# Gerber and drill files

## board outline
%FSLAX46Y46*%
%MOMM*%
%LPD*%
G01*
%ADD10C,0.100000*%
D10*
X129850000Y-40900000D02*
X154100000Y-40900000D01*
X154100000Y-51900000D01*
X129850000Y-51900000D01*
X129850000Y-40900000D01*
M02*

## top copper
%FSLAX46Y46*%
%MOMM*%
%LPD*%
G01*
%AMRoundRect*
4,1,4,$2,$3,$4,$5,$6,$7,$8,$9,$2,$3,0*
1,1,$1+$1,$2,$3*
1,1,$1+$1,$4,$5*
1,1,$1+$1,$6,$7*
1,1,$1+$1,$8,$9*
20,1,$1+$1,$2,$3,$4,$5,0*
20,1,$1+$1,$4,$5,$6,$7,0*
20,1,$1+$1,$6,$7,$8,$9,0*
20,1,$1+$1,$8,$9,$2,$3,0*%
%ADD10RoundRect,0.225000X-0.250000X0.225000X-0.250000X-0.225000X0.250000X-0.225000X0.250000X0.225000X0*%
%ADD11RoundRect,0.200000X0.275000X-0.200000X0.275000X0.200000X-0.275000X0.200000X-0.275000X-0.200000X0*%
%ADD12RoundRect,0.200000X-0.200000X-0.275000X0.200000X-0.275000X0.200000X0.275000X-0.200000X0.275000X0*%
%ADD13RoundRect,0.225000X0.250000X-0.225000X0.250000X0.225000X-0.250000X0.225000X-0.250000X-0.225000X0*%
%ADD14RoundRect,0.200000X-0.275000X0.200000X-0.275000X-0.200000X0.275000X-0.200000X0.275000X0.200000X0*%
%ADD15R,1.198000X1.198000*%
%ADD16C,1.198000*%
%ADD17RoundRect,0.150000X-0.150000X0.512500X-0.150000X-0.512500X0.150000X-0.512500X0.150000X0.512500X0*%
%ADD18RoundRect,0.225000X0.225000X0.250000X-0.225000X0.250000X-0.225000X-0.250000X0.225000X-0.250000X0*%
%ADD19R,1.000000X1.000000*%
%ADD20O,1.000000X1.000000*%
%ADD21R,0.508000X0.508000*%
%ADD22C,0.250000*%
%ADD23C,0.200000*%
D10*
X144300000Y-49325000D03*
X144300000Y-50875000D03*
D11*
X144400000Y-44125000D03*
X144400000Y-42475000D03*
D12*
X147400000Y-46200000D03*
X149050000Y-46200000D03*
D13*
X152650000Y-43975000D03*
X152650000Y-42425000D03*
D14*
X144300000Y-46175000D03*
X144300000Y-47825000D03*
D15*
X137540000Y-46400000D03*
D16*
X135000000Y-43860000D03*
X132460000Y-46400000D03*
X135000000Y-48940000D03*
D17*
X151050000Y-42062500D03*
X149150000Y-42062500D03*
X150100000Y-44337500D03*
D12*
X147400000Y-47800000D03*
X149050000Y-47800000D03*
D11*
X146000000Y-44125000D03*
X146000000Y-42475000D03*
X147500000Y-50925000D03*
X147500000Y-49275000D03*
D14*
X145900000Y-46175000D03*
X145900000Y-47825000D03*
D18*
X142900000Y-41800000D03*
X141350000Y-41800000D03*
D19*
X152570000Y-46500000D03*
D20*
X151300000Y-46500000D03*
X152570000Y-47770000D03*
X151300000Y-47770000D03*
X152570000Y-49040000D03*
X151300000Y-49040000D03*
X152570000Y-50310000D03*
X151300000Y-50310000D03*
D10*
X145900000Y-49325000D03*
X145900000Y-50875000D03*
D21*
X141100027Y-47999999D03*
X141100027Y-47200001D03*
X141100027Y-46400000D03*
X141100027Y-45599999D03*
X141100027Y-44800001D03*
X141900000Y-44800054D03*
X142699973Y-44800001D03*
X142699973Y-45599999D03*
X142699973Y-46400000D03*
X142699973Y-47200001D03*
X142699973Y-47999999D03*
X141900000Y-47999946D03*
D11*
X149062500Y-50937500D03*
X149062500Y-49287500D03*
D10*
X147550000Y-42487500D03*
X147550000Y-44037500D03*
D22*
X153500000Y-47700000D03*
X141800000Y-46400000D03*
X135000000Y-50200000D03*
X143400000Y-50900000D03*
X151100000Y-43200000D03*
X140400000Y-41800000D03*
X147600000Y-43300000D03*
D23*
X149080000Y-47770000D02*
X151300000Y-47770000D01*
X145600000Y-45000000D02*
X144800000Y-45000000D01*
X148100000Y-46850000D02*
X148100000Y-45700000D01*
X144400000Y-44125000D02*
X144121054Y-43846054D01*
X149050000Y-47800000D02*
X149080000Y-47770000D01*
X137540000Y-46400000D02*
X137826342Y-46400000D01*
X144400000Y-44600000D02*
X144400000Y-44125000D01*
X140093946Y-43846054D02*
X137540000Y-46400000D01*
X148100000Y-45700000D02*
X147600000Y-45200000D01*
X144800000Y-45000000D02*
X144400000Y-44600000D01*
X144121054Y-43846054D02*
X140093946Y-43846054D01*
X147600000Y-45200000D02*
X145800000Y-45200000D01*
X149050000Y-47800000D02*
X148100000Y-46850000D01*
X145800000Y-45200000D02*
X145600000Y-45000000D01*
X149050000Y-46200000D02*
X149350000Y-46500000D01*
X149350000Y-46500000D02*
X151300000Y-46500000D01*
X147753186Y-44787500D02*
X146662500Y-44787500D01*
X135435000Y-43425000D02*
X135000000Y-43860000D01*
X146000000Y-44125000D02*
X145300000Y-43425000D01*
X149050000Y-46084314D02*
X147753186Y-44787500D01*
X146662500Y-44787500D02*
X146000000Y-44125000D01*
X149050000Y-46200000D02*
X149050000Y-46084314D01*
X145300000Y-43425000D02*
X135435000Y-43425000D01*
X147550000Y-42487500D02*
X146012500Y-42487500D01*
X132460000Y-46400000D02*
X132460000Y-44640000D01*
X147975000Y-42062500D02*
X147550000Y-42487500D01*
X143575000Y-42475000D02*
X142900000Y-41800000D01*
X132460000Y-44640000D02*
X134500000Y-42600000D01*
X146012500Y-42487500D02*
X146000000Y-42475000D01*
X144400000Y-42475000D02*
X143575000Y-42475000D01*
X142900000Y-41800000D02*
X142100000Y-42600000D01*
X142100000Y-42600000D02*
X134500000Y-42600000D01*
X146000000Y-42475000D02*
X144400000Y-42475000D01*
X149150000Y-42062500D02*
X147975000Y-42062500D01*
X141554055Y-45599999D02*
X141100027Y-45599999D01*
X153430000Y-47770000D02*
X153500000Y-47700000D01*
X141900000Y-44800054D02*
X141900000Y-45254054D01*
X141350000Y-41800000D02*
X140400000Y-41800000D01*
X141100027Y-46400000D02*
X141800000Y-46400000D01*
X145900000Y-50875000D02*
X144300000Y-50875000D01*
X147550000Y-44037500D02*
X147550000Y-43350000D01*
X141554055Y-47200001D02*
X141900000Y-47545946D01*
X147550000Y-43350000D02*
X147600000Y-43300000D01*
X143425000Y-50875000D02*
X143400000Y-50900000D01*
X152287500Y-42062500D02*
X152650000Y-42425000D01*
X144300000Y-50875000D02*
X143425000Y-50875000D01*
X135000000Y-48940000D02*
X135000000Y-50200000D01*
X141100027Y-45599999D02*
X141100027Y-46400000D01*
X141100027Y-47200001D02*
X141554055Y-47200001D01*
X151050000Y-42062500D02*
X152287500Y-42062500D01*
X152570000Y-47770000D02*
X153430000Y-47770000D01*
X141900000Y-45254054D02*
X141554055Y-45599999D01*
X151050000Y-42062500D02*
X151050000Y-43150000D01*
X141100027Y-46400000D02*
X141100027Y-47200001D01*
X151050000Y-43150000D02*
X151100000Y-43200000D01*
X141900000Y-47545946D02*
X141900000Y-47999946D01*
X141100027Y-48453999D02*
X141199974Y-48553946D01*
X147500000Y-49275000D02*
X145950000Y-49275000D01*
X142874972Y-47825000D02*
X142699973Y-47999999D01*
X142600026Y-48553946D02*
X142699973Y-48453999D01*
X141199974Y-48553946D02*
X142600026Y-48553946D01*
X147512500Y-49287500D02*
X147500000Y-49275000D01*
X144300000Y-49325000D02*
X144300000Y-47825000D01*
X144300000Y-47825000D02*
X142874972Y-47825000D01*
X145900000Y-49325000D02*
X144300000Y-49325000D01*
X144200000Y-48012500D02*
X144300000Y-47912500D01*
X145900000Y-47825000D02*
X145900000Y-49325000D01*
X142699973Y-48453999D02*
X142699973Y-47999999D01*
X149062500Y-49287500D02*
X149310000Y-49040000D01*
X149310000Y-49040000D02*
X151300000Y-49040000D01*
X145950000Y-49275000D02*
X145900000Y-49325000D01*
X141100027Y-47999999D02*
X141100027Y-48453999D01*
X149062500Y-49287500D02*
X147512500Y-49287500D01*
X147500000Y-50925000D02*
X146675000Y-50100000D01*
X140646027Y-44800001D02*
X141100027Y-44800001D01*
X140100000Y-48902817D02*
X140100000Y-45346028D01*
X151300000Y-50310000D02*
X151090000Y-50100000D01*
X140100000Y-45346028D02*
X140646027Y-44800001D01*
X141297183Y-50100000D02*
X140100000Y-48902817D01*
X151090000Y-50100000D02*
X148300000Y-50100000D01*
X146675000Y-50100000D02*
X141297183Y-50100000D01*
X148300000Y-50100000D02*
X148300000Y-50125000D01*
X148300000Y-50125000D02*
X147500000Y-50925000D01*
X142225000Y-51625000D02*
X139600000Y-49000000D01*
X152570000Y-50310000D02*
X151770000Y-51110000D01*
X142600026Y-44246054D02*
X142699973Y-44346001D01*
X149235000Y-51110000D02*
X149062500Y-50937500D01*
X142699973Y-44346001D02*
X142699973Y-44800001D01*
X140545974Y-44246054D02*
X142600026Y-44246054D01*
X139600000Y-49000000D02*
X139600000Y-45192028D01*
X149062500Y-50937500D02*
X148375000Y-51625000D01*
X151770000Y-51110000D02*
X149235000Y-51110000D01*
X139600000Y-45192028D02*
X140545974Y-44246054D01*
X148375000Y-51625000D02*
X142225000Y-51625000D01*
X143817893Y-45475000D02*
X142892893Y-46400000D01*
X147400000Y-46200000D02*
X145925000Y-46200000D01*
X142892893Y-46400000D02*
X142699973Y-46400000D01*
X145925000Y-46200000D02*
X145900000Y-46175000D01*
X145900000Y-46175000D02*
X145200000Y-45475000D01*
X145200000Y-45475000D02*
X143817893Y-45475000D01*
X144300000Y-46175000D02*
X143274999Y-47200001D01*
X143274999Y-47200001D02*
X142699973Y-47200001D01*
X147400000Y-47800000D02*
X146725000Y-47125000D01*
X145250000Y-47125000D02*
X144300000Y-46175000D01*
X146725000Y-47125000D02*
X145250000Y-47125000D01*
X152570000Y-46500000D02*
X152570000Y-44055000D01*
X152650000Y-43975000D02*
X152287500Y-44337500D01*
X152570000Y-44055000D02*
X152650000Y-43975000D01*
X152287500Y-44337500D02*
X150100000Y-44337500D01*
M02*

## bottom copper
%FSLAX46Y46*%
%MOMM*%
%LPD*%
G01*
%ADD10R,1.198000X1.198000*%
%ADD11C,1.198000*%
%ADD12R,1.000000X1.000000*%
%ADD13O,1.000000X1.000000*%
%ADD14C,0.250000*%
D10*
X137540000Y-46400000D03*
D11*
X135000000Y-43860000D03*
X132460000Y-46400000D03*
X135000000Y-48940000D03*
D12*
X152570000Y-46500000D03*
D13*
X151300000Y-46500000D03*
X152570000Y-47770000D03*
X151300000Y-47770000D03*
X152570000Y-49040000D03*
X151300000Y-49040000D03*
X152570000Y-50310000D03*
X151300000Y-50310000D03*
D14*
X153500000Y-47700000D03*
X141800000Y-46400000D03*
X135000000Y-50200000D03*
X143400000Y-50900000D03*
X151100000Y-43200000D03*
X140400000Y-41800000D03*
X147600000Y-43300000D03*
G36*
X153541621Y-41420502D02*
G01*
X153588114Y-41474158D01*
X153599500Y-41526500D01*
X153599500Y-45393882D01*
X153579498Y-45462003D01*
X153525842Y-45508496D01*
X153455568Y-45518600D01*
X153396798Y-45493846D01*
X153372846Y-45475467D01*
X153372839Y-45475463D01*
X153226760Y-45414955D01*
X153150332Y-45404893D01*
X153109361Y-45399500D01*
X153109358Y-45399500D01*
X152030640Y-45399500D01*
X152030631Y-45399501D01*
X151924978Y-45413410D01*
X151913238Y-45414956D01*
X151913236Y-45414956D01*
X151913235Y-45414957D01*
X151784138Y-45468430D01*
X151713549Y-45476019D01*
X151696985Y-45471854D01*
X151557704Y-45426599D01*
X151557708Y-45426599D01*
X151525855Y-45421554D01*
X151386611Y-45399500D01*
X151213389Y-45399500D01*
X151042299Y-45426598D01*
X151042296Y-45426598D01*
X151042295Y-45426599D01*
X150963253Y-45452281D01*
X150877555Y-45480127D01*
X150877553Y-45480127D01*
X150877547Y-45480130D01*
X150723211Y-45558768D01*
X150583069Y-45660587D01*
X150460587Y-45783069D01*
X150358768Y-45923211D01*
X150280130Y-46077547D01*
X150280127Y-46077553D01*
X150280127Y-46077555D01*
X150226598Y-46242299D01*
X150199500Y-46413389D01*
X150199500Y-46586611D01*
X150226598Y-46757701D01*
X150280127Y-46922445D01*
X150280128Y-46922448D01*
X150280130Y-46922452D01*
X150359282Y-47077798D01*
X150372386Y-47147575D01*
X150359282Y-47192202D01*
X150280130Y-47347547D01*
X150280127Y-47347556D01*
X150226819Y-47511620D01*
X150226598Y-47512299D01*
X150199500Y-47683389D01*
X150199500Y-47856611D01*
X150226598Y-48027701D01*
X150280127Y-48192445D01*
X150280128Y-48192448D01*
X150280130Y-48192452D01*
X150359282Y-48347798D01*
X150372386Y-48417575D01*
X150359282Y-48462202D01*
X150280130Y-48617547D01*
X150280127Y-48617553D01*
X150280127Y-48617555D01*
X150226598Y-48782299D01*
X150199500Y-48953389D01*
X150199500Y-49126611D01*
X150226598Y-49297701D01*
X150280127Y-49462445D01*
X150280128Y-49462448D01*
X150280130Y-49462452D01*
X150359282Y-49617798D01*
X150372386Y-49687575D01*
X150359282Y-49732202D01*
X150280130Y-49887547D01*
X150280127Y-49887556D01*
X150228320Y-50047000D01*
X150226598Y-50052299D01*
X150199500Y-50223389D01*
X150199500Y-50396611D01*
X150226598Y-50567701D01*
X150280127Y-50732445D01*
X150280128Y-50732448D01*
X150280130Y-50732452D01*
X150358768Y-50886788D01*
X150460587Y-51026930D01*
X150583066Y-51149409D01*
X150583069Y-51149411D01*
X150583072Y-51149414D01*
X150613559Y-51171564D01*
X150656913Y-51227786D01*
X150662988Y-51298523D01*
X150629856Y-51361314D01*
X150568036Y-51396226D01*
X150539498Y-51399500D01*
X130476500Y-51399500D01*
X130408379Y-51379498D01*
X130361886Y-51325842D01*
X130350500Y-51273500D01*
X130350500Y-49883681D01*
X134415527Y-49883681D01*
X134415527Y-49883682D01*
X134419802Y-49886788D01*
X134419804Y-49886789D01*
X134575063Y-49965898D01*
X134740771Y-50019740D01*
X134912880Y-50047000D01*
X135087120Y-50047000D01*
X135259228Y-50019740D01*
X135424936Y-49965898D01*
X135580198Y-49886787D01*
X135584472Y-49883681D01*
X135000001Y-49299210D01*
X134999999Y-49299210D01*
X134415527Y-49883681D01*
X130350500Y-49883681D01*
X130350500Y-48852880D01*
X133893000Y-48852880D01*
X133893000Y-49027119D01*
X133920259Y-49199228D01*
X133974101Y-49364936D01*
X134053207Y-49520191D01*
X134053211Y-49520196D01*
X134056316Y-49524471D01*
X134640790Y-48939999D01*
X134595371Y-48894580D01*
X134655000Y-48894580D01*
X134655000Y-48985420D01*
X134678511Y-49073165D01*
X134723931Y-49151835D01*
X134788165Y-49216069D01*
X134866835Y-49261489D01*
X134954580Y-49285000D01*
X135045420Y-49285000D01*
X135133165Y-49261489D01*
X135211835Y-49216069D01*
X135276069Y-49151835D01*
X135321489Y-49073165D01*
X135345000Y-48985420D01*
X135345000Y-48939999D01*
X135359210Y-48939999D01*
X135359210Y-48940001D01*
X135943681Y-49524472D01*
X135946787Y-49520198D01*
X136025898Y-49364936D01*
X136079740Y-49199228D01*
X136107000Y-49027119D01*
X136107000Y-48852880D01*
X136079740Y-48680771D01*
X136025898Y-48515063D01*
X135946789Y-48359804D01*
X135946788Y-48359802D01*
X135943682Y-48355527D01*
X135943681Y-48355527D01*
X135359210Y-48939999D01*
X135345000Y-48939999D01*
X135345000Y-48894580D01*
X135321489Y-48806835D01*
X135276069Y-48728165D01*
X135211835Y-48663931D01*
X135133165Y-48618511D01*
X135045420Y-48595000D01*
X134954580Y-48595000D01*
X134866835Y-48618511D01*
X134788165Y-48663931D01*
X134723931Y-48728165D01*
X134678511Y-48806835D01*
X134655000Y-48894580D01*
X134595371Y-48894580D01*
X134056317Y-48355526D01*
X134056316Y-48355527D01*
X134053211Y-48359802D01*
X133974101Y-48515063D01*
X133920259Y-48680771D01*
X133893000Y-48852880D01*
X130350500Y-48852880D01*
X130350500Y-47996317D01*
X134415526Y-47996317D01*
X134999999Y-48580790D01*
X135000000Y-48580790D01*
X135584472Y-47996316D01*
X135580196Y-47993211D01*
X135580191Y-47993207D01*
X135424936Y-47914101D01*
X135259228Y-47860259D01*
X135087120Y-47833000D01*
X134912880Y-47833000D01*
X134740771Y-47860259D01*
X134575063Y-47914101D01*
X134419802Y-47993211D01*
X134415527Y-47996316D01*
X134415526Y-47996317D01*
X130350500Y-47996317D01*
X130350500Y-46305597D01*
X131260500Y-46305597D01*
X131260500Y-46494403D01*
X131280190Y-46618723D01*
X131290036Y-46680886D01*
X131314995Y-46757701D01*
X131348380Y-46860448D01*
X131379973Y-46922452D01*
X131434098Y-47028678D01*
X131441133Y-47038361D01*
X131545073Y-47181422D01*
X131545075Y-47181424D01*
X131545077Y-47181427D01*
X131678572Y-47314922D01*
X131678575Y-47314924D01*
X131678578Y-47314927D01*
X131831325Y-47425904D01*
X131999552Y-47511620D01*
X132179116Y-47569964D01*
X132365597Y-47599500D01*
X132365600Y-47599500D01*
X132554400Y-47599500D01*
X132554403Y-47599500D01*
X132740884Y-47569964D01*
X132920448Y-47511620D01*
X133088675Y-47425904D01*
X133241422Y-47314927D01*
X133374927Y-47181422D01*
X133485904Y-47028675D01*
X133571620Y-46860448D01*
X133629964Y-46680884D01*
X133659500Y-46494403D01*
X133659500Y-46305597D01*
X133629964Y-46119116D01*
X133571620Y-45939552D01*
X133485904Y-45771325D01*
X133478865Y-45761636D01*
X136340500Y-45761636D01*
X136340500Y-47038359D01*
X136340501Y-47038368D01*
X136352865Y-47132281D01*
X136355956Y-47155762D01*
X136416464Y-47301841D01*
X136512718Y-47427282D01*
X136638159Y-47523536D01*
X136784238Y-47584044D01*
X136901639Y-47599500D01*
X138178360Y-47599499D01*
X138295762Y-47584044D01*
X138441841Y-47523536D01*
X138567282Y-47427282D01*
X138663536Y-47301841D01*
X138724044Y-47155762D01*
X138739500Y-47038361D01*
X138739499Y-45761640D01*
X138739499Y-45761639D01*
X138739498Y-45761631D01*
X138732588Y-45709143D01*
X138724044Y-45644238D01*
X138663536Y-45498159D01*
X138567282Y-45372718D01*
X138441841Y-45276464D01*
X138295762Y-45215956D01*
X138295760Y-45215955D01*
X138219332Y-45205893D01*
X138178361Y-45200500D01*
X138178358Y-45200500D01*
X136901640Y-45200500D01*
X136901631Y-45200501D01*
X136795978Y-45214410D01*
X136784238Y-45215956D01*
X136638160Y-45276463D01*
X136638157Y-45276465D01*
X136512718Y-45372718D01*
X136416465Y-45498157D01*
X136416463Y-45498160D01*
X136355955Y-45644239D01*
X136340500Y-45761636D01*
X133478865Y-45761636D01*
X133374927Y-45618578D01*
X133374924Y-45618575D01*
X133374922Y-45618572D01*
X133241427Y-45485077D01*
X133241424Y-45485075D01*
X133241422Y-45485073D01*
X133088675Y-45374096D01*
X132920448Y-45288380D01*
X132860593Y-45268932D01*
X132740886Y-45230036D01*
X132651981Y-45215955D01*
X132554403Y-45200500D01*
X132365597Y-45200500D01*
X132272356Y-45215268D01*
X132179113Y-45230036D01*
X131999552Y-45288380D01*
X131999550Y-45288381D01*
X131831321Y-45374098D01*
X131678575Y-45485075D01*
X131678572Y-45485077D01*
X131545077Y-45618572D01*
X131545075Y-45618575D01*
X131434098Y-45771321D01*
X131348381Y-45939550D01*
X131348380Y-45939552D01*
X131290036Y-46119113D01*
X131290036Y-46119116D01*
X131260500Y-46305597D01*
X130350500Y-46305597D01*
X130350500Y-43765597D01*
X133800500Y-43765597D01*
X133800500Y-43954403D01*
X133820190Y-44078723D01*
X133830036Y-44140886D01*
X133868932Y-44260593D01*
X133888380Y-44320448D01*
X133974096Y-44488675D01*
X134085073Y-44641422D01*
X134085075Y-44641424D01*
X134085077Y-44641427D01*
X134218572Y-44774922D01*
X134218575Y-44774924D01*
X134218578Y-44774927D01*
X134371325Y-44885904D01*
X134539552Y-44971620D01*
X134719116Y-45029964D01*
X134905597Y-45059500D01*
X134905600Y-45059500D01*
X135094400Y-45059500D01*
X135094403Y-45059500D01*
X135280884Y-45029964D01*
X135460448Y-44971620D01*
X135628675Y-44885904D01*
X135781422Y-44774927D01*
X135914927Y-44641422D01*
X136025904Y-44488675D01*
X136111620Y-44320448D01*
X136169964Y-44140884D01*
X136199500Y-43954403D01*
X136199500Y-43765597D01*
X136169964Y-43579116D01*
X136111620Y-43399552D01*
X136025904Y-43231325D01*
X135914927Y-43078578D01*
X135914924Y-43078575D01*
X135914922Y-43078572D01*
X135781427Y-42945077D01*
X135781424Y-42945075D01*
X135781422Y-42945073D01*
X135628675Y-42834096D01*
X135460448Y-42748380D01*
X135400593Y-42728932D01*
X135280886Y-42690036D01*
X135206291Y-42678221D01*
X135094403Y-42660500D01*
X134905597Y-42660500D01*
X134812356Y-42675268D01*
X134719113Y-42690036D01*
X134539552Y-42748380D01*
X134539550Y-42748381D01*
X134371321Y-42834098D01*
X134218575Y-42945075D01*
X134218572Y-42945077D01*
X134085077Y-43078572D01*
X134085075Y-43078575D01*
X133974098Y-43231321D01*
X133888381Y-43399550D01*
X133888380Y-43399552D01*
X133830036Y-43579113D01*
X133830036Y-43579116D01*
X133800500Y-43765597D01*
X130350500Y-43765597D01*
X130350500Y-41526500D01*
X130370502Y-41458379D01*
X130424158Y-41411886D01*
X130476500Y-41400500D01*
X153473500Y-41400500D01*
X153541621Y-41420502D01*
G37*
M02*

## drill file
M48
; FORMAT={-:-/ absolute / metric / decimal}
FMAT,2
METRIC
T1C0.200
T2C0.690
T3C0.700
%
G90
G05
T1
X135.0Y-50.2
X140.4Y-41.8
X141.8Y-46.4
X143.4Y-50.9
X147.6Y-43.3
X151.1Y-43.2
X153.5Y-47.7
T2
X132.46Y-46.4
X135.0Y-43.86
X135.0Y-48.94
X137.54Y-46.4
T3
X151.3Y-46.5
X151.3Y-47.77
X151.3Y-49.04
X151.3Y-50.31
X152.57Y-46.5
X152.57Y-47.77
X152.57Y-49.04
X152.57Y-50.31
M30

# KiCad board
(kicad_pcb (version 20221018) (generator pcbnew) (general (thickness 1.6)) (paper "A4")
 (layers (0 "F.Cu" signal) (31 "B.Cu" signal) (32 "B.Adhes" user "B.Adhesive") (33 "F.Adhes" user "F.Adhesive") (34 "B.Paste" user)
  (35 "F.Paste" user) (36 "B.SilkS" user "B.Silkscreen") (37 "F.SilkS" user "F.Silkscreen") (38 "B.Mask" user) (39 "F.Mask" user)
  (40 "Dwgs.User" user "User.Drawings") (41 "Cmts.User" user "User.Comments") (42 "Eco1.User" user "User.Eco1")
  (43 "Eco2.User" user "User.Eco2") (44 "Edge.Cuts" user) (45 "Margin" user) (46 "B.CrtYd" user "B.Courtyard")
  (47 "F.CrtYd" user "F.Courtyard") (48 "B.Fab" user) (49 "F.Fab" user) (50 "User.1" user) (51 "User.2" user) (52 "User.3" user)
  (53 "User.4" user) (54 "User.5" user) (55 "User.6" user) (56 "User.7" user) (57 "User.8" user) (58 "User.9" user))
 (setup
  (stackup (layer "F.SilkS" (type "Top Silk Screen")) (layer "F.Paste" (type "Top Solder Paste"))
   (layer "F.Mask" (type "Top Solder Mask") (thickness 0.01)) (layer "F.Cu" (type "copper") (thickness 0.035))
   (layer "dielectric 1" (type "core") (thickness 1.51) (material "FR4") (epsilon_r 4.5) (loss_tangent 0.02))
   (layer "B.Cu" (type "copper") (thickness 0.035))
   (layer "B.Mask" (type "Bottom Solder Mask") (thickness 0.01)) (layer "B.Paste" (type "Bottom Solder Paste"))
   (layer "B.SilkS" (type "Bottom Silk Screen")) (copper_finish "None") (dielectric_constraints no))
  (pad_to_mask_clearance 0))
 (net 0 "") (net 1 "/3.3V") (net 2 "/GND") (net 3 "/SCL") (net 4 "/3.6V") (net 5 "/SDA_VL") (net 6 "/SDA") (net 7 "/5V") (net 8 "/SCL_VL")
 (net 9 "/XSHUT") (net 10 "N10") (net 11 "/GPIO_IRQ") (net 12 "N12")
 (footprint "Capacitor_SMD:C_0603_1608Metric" (layer "F.Cu") (at 144.3 50.1 -90)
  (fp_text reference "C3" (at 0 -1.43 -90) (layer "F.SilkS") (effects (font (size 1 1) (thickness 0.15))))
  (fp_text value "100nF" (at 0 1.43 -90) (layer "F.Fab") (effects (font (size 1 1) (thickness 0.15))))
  (pad "1" smd roundrect (at -0.775 0 270) (size 0.9 0.95) (layers "F.Cu" "F.Paste" "F.Mask") (roundrect_rratio 0.25) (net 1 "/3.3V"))
  (pad "2" smd roundrect (at 0.775 0 270) (size 0.9 0.95) (layers "F.Cu" "F.Paste" "F.Mask") (roundrect_rratio 0.25) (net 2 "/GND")))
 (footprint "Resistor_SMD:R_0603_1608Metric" (layer "F.Cu") (at 144.4 43.3 90)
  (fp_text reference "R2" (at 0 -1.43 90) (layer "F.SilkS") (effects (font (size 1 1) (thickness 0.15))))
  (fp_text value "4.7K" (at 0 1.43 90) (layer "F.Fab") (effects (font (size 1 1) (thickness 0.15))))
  (pad "1" smd roundrect (at -0.825 0 90) (size 0.8 0.95) (layers "F.Cu" "F.Paste" "F.Mask") (roundrect_rratio 0.25) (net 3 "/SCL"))
  (pad "2" smd roundrect (at 0.825 0 90) (size 0.8 0.95) (layers "F.Cu" "F.Paste" "F.Mask") (roundrect_rratio 0.25) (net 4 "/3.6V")))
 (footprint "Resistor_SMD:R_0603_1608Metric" (layer "F.Cu") (at 148.225 46.2)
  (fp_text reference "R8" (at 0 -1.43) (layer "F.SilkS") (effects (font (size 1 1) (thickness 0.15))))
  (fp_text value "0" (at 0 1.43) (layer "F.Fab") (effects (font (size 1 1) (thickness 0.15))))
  (pad "1" smd roundrect (at -0.825 0) (size 0.8 0.95) (layers "F.Cu" "F.Paste" "F.Mask") (roundrect_rratio 0.25) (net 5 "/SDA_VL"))
  (pad "2" smd roundrect (at 0.825 0) (size 0.8 0.95) (layers "F.Cu" "F.Paste" "F.Mask") (roundrect_rratio 0.25) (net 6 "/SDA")))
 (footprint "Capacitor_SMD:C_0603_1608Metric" (layer "F.Cu") (at 152.65 43.2 90)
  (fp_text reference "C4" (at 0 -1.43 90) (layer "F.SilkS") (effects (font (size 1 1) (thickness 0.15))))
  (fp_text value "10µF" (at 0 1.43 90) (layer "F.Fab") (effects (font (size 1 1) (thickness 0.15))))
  (pad "1" smd roundrect (at -0.775 0 90) (size 0.9 0.95) (layers "F.Cu" "F.Paste" "F.Mask") (roundrect_rratio 0.25) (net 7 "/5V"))
  (pad "2" smd roundrect (at 0.775 0 90) (size 0.9 0.95) (layers "F.Cu" "F.Paste" "F.Mask") (roundrect_rratio 0.25) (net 2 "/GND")))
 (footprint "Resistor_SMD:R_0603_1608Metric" (layer "F.Cu") (at 144.3 47 -90)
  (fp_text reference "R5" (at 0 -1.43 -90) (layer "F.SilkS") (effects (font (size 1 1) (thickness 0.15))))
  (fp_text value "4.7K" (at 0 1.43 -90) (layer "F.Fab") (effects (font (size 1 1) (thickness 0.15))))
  (pad "1" smd roundrect (at -0.825 0 270) (size 0.8 0.95) (layers "F.Cu" "F.Paste" "F.Mask") (roundrect_rratio 0.25) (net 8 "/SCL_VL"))
  (pad "2" smd roundrect (at 0.825 0 270) (size 0.8 0.95) (layers "F.Cu" "F.Paste" "F.Mask") (roundrect_rratio 0.25) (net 1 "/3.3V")))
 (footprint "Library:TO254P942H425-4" (layer "F.Cu") (at 135 46.4 180)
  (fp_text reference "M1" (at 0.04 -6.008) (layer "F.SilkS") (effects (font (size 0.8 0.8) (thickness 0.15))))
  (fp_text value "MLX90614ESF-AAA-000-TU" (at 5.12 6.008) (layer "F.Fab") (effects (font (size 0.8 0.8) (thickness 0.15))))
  (pad "1" thru_hole rect (at -2.54 0 180) (size 1.198 1.198) (drill 0.69) (layers "*.Cu" "*.Mask") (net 3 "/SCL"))
  (pad "2" thru_hole circle (at 0 2.54 180) (size 1.198 1.198) (drill 0.69) (layers "*.Cu" "*.Mask") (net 6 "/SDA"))
  (pad "3" thru_hole circle (at 2.54 0 180) (size 1.198 1.198) (drill 0.69) (layers "*.Cu" "*.Mask") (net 4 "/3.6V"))
  (pad "4" thru_hole circle (at 0 -2.54 180) (size 1.198 1.198) (drill 0.69) (layers "*.Cu" "*.Mask") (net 2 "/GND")))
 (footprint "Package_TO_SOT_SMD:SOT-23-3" (layer "F.Cu") (at 150.1 43.2 -90)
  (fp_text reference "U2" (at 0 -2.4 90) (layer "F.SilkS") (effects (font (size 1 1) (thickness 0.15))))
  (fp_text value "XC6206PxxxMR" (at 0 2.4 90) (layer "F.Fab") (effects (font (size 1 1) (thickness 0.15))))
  (pad "1" smd roundrect (at -1.1375 -0.95 270) (size 1.325 0.6) (layers "F.Cu" "F.Paste" "F.Mask") (roundrect_rratio 0.25) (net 2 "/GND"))
  (pad "2" smd roundrect (at -1.1375 0.95 270) (size 1.325 0.6) (layers "F.Cu" "F.Paste" "F.Mask") (roundrect_rratio 0.25) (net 4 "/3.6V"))
  (pad "3" smd roundrect (at 1.1375 0 270) (size 1.325 0.6) (layers "F.Cu" "F.Paste" "F.Mask") (roundrect_rratio 0.25) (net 7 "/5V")))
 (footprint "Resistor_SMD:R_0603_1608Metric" (layer "F.Cu") (at 148.225 47.8)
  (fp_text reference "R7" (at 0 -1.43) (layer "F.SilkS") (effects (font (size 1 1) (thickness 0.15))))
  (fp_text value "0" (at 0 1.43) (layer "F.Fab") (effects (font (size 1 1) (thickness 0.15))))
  (pad "1" smd roundrect (at -0.825 0) (size 0.8 0.95) (layers "F.Cu" "F.Paste" "F.Mask") (roundrect_rratio 0.25) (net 8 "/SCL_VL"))
  (pad "2" smd roundrect (at 0.825 0) (size 0.8 0.95) (layers "F.Cu" "F.Paste" "F.Mask") (roundrect_rratio 0.25) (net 3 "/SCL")))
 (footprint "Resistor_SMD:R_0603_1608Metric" (layer "F.Cu") (at 146 43.3 90)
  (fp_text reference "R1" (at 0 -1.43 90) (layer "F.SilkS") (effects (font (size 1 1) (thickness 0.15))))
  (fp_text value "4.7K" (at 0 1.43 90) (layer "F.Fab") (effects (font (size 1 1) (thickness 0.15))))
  (pad "1" smd roundrect (at -0.825 0 90) (size 0.8 0.95) (layers "F.Cu" "F.Paste" "F.Mask") (roundrect_rratio 0.25) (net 6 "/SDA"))
  (pad "2" smd roundrect (at 0.825 0 90) (size 0.8 0.95) (layers "F.Cu" "F.Paste" "F.Mask") (roundrect_rratio 0.25) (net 4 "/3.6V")))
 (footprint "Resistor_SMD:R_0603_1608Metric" (layer "F.Cu") (at 147.5 50.1 90)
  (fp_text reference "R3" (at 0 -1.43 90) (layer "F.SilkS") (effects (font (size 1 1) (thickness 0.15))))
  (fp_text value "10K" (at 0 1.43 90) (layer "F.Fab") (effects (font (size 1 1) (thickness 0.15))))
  (pad "1" smd roundrect (at -0.825 0 90) (size 0.8 0.95) (layers "F.Cu" "F.Paste" "F.Mask") (roundrect_rratio 0.25) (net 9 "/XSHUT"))
  (pad "2" smd roundrect (at 0.825 0 90) (size 0.8 0.95) (layers "F.Cu" "F.Paste" "F.Mask") (roundrect_rratio 0.25) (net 1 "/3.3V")))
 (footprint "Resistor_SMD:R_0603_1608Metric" (layer "F.Cu") (at 145.9 47 -90)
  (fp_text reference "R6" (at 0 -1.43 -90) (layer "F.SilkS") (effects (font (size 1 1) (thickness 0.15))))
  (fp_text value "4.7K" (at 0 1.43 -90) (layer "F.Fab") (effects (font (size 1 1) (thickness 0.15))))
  (pad "1" smd roundrect (at -0.825 0 270) (size 0.8 0.95) (layers "F.Cu" "F.Paste" "F.Mask") (roundrect_rratio 0.25) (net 5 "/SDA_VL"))
  (pad "2" smd roundrect (at 0.825 0 270) (size 0.8 0.95) (layers "F.Cu" "F.Paste" "F.Mask") (roundrect_rratio 0.25) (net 1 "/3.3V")))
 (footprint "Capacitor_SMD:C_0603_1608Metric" (layer "F.Cu") (at 142.125 41.8 180)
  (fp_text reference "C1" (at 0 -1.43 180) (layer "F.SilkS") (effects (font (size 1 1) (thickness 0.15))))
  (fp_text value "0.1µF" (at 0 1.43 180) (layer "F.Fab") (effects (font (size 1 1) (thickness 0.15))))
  (pad "1" smd roundrect (at -0.775 0 180) (size 0.9 0.95) (layers "F.Cu" "F.Paste" "F.Mask") (roundrect_rratio 0.25) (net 4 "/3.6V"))
  (pad "2" smd roundrect (at 0.775 0 180) (size 0.9 0.95) (layers "F.Cu" "F.Paste" "F.Mask") (roundrect_rratio 0.25) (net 2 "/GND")))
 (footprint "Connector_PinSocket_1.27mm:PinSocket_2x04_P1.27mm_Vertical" (layer "F.Cu") (at 152.57 46.5)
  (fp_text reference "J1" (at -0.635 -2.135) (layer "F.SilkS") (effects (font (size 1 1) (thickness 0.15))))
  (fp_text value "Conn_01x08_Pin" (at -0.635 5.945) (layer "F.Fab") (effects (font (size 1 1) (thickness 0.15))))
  (pad "1" thru_hole rect (at 0 0) (size 1 1) (drill 0.7) (layers "*.Cu" "*.Mask") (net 7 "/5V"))
  (pad "2" thru_hole oval (at -1.27 0) (size 1 1) (drill 0.7) (layers "*.Cu" "*.Mask") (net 6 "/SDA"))
  (pad "3" thru_hole oval (at 0 1.27) (size 1 1) (drill 0.7) (layers "*.Cu" "*.Mask") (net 2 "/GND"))
  (pad "4" thru_hole oval (at -1.27 1.27) (size 1 1) (drill 0.7) (layers "*.Cu" "*.Mask") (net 3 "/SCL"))
  (pad "5" thru_hole oval (at 0 2.54) (size 1 1) (drill 0.7) (layers "*.Cu" "*.Mask") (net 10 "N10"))
  (pad "6" thru_hole oval (at -1.27 2.54) (size 1 1) (drill 0.7) (layers "*.Cu" "*.Mask") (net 1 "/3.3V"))
  (pad "7" thru_hole oval (at 0 3.81) (size 1 1) (drill 0.7) (layers "*.Cu" "*.Mask") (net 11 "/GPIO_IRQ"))
  (pad "8" thru_hole oval (at -1.27 3.81) (size 1 1) (drill 0.7) (layers "*.Cu" "*.Mask") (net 9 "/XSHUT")))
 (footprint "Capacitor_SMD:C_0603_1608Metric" (layer "F.Cu") (at 145.9 50.1 -90)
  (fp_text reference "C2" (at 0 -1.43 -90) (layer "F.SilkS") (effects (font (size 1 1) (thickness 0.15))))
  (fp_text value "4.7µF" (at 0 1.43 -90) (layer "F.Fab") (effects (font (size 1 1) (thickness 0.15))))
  (pad "1" smd roundrect (at -0.775 0 270) (size 0.9 0.95) (layers "F.Cu" "F.Paste" "F.Mask") (roundrect_rratio 0.25) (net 1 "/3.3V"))
  (pad "2" smd roundrect (at 0.775 0 270) (size 0.9 0.95) (layers "F.Cu" "F.Paste" "F.Mask") (roundrect_rratio 0.25) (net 2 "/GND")))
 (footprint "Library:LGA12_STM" (layer "F.Cu") (at 141.9 46.4 180)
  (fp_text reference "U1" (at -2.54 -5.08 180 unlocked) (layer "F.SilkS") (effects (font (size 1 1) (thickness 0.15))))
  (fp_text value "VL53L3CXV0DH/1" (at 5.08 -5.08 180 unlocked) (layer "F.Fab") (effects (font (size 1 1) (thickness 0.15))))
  (pad "1" smd rect (at 0.799973 -1.599999 270) (size 0.508 0.508) (layers "F.Cu" "F.Paste" "F.Mask") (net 1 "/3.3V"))
  (pad "2" smd rect (at 0.799973 -0.800001 270) (size 0.508 0.508) (layers "F.Cu" "F.Paste" "F.Mask") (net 2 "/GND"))
  (pad "3" smd rect (at 0.799973 0 270) (size 0.508 0.508) (layers "F.Cu" "F.Paste" "F.Mask") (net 2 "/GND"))
  (pad "4" smd rect (at 0.799973 0.800001 270) (size 0.508 0.508) (layers "F.Cu" "F.Paste" "F.Mask") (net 2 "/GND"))
  (pad "5" smd rect (at 0.799973 1.599999 270) (size 0.508 0.508) (layers "F.Cu" "F.Paste" "F.Mask") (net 9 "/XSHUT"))
  (pad "6" smd rect (at 0 1.599946 180) (size 0.508 0.508) (layers "F.Cu" "F.Paste" "F.Mask") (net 2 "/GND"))
  (pad "7" smd rect (at -0.799973 1.599999 270) (size 0.508 0.508) (layers "F.Cu" "F.Paste" "F.Mask") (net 11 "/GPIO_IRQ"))
  (pad "8" smd rect (at -0.799973 0.800001 270) (size 0.508 0.508) (layers "F.Cu" "F.Paste" "F.Mask") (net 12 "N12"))
  (pad "9" smd rect (at -0.799973 0 270) (size 0.508 0.508) (layers "F.Cu" "F.Paste" "F.Mask") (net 5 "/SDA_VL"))
  (pad "10" smd rect (at -0.799973 -0.800001 270) (size 0.508 0.508) (layers "F.Cu" "F.Paste" "F.Mask") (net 8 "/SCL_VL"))
  (pad "11" smd rect (at -0.799973 -1.599999 270) (size 0.508 0.508) (layers "F.Cu" "F.Paste" "F.Mask") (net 1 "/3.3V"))
  (pad "12" smd rect (at 0 -1.599946 180) (size 0.508 0.508) (layers "F.Cu" "F.Paste" "F.Mask") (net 2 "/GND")))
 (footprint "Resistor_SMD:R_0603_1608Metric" (layer "F.Cu") (at 149.0625 50.1125 90)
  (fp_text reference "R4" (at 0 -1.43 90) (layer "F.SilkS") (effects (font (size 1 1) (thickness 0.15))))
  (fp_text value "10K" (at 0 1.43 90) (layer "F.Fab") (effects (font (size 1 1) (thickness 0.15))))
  (pad "1" smd roundrect (at -0.825 0 90) (size 0.8 0.95) (layers "F.Cu" "F.Paste" "F.Mask") (roundrect_rratio 0.25) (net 11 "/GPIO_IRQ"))
  (pad "2" smd roundrect (at 0.825 0 90) (size 0.8 0.95) (layers "F.Cu" "F.Paste" "F.Mask") (roundrect_rratio 0.25) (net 1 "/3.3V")))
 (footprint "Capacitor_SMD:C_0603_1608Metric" (layer "F.Cu") (at 147.55 43.2625 -90)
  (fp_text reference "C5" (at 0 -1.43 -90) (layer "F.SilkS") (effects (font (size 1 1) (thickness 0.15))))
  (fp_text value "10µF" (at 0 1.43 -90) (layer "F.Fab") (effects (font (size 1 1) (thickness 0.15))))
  (pad "1" smd roundrect (at -0.775 0 270) (size 0.9 0.95) (layers "F.Cu" "F.Paste" "F.Mask") (roundrect_rratio 0.25) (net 4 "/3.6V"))
  (pad "2" smd roundrect (at 0.775 0 270) (size 0.9 0.95) (layers "F.Cu" "F.Paste" "F.Mask") (roundrect_rratio 0.25) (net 2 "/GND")))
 (gr_rect (start 129.85 40.9) (end 154.1 51.9) (stroke (width 0.1) (type default)) (fill none) (layer "Edge.Cuts"))
 (segment (start 149.08 47.77) (end 151.3 47.77) (width 0.2) (layer "F.Cu") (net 3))
 (segment (start 145.6 45) (end 144.8 45) (width 0.2) (layer "F.Cu") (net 3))
 (segment (start 148.1 46.85) (end 148.1 45.7) (width 0.2) (layer "F.Cu") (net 3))
 (segment (start 144.4 44.125) (end 144.121054 43.846054) (width 0.2) (layer "F.Cu") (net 3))
 (segment (start 149.05 47.8) (end 149.08 47.77) (width 0.2) (layer "F.Cu") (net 3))
 (segment (start 137.54 46.4) (end 137.826342 46.4) (width 0.2) (layer "F.Cu") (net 3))
 (segment (start 144.4 44.6) (end 144.4 44.125) (width 0.2) (layer "F.Cu") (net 3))
 (segment (start 140.093946 43.846054) (end 137.54 46.4) (width 0.2) (layer "F.Cu") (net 3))
 (segment (start 148.1 45.7) (end 147.6 45.2) (width 0.2) (layer "F.Cu") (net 3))
 (segment (start 144.8 45) (end 144.4 44.6) (width 0.2) (layer "F.Cu") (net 3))
 (segment (start 144.121054 43.846054) (end 140.093946 43.846054) (width 0.2) (layer "F.Cu") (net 3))
 (segment (start 147.6 45.2) (end 145.8 45.2) (width 0.2) (layer "F.Cu") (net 3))
 (segment (start 149.05 47.8) (end 148.1 46.85) (width 0.2) (layer "F.Cu") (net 3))
 (segment (start 145.8 45.2) (end 145.6 45) (width 0.2) (layer "F.Cu") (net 3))
 (segment (start 149.05 46.2) (end 149.35 46.5) (width 0.2) (layer "F.Cu") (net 6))
 (segment (start 149.35 46.5) (end 151.3 46.5) (width 0.2) (layer "F.Cu") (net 6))
 (segment (start 147.753186 44.7875) (end 146.6625 44.7875) (width 0.2) (layer "F.Cu") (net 6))
 (segment (start 135.435 43.425) (end 135 43.86) (width 0.2) (layer "F.Cu") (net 6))
 (segment (start 146 44.125) (end 145.3 43.425) (width 0.2) (layer "F.Cu") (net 6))
 (segment (start 149.05 46.084314) (end 147.753186 44.7875) (width 0.2) (layer "F.Cu") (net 6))
 (segment (start 146.6625 44.7875) (end 146 44.125) (width 0.2) (layer "F.Cu") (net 6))
 (segment (start 149.05 46.2) (end 149.05 46.084314) (width 0.2) (layer "F.Cu") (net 6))
 (segment (start 145.3 43.425) (end 135.435 43.425) (width 0.2) (layer "F.Cu") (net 6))
 (segment (start 147.55 42.4875) (end 146.0125 42.4875) (width 0.2) (layer "F.Cu") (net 4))
 (segment (start 132.46 46.4) (end 132.46 44.64) (width 0.2) (layer "F.Cu") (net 4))
 (segment (start 147.975 42.0625) (end 147.55 42.4875) (width 0.2) (layer "F.Cu") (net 4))
 (segment (start 143.575 42.475) (end 142.9 41.8) (width 0.2) (layer "F.Cu") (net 4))
 (segment (start 132.46 44.64) (end 134.5 42.6) (width 0.2) (layer "F.Cu") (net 4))
 (segment (start 146.0125 42.4875) (end 146 42.475) (width 0.2) (layer "F.Cu") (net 4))
 (segment (start 144.4 42.475) (end 143.575 42.475) (width 0.2) (layer "F.Cu") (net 4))
 (segment (start 142.9 41.8) (end 142.1 42.6) (width 0.2) (layer "F.Cu") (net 4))
 (segment (start 142.1 42.6) (end 134.5 42.6) (width 0.2) (layer "F.Cu") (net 4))
 (segment (start 146 42.475) (end 144.4 42.475) (width 0.2) (layer "F.Cu") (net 4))
 (segment (start 149.15 42.0625) (end 147.975 42.0625) (width 0.2) (layer "F.Cu") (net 4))
 (segment (start 141.554055 45.599999) (end 141.100027 45.599999) (width 0.2) (layer "F.Cu") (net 2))
 (segment (start 153.43 47.77) (end 153.5 47.7) (width 0.2) (layer "F.Cu") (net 2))
 (segment (start 141.9 44.800054) (end 141.9 45.254054) (width 0.2) (layer "F.Cu") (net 2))
 (segment (start 141.35 41.8) (end 140.4 41.8) (width 0.2) (layer "F.Cu") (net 2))
 (segment (start 141.100027 46.4) (end 141.8 46.4) (width 0.2) (layer "F.Cu") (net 2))
 (segment (start 145.9 50.875) (end 144.3 50.875) (width 0.2) (layer "F.Cu") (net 2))
 (segment (start 147.55 44.0375) (end 147.55 43.35) (width 0.2) (layer "F.Cu") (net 2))
 (segment (start 141.554055 47.200001) (end 141.9 47.545946) (width 0.2) (layer "F.Cu") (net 2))
 (segment (start 147.55 43.35) (end 147.6 43.3) (width 0.2) (layer "F.Cu") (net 2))
 (segment (start 143.425 50.875) (end 143.4 50.9) (width 0.2) (layer "F.Cu") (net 2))
 (segment (start 152.2875 42.0625) (end 152.65 42.425) (width 0.2) (layer "F.Cu") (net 2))
 (segment (start 144.3 50.875) (end 143.425 50.875) (width 0.2) (layer "F.Cu") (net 2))
 (segment (start 135 48.94) (end 135 50.2) (width 0.2) (layer "F.Cu") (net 2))
 (segment (start 141.100027 45.599999) (end 141.100027 46.4) (width 0.2) (layer "F.Cu") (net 2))
 (segment (start 141.100027 47.200001) (end 141.554055 47.200001) (width 0.2) (layer "F.Cu") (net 2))
 (segment (start 151.05 42.0625) (end 152.2875 42.0625) (width 0.2) (layer "F.Cu") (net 2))
 (segment (start 152.57 47.77) (end 153.43 47.77) (width 0.2) (layer "F.Cu") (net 2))
 (segment (start 141.9 45.254054) (end 141.554055 45.599999) (width 0.2) (layer "F.Cu") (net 2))
 (segment (start 151.05 42.0625) (end 151.05 43.15) (width 0.2) (layer "F.Cu") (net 2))
 (segment (start 141.100027 46.4) (end 141.100027 47.200001) (width 0.2) (layer "F.Cu") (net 2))
 (segment (start 151.05 43.15) (end 151.1 43.2) (width 0.2) (layer "F.Cu") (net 2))
 (segment (start 141.9 47.545946) (end 141.9 47.999946) (width 0.2) (layer "F.Cu") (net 2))
 (via (at 153.5 47.7) (size 0.25) (drill 0.2) (layers "F.Cu" "B.Cu") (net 2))
 (via (at 141.8 46.4) (size 0.25) (drill 0.2) (layers "F.Cu" "B.Cu") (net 2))
 (via (at 135 50.2) (size 0.25) (drill 0.2) (layers "F.Cu" "B.Cu") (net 2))
 (via (at 143.4 50.9) (size 0.25) (drill 0.2) (layers "F.Cu" "B.Cu") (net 2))
 (via (at 151.1 43.2) (size 0.25) (drill 0.2) (layers "F.Cu" "B.Cu") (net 2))
 (via (at 140.4 41.8) (size 0.25) (drill 0.2) (layers "F.Cu" "B.Cu") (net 2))
 (via (at 147.6 43.3) (size 0.25) (drill 0.2) (layers "F.Cu" "B.Cu") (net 2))
 (segment (start 141.100027 48.453999) (end 141.199974 48.553946) (width 0.2) (layer "F.Cu") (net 1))
 (segment (start 147.5 49.275) (end 145.95 49.275) (width 0.2) (layer "F.Cu") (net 1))
 (segment (start 142.874972 47.825) (end 142.699973 47.999999) (width 0.2) (layer "F.Cu") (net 1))
 (segment (start 142.600026 48.553946) (end 142.699973 48.453999) (width 0.2) (layer "F.Cu") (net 1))
 (segment (start 141.199974 48.553946) (end 142.600026 48.553946) (width 0.2) (layer "F.Cu") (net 1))
 (segment (start 147.5125 49.2875) (end 147.5 49.275) (width 0.2) (layer "F.Cu") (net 1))
 (segment (start 144.3 49.325) (end 144.3 47.825) (width 0.2) (layer "F.Cu") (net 1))
 (segment (start 144.3 47.825) (end 142.874972 47.825) (width 0.2) (layer "F.Cu") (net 1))
 (segment (start 145.9 49.325) (end 144.3 49.325) (width 0.2) (layer "F.Cu") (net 1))
 (segment (start 144.2 48.0125) (end 144.3 47.9125) (width 0.2) (layer "F.Cu") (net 1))
 (segment (start 145.9 47.825) (end 145.9 49.325) (width 0.2) (layer "F.Cu") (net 1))
 (segment (start 142.699973 48.453999) (end 142.699973 47.999999) (width 0.2) (layer "F.Cu") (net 1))
 (segment (start 149.0625 49.2875) (end 149.31 49.04) (width 0.2) (layer "F.Cu") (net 1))
 (segment (start 149.31 49.04) (end 151.3 49.04) (width 0.2) (layer "F.Cu") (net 1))
 (segment (start 145.95 49.275) (end 145.9 49.325) (width 0.2) (layer "F.Cu") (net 1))
 (segment (start 141.100027 47.999999) (end 141.100027 48.453999) (width 0.2) (layer "F.Cu") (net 1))
 (segment (start 149.0625 49.2875) (end 147.5125 49.2875) (width 0.2) (layer "F.Cu") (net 1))
 (segment (start 147.5 50.925) (end 146.675 50.1) (width 0.2) (layer "F.Cu") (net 9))
 (segment (start 140.646027 44.800001) (end 141.100027 44.800001) (width 0.2) (layer "F.Cu") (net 9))
 (segment (start 140.1 48.902817) (end 140.1 45.346028) (width 0.2) (layer "F.Cu") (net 9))
 (segment (start 151.3 50.31) (end 151.09 50.1) (width 0.2) (layer "F.Cu") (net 9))
 (segment (start 140.1 45.346028) (end 140.646027 44.800001) (width 0.2) (layer "F.Cu") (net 9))
 (segment (start 141.297183 50.1) (end 140.1 48.902817) (width 0.2) (layer "F.Cu") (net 9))
 (segment (start 151.09 50.1) (end 148.3 50.1) (width 0.2) (layer "F.Cu") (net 9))
 (segment (start 146.675 50.1) (end 141.297183 50.1) (width 0.2) (layer "F.Cu") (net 9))
 (segment (start 148.3 50.1) (end 148.3 50.125) (width 0.2) (layer "F.Cu") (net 9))
 (segment (start 148.3 50.125) (end 147.5 50.925) (width 0.2) (layer "F.Cu") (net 9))
 (segment (start 142.225 51.625) (end 139.6 49) (width 0.2) (layer "F.Cu") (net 11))
 (segment (start 152.57 50.31) (end 151.77 51.11) (width 0.2) (layer "F.Cu") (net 11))
 (segment (start 142.600026 44.246054) (end 142.699973 44.346001) (width 0.2) (layer "F.Cu") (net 11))
 (segment (start 149.235 51.11) (end 149.0625 50.9375) (width 0.2) (layer "F.Cu") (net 11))
 (segment (start 142.699973 44.346001) (end 142.699973 44.800001) (width 0.2) (layer "F.Cu") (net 11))
 (segment (start 140.545974 44.246054) (end 142.600026 44.246054) (width 0.2) (layer "F.Cu") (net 11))
 (segment (start 139.6 49) (end 139.6 45.192028) (width 0.2) (layer "F.Cu") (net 11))
 (segment (start 149.0625 50.9375) (end 148.375 51.625) (width 0.2) (layer "F.Cu") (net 11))
 (segment (start 151.77 51.11) (end 149.235 51.11) (width 0.2) (layer "F.Cu") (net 11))
 (segment (start 139.6 45.192028) (end 140.545974 44.246054) (width 0.2) (layer "F.Cu") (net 11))
 (segment (start 148.375 51.625) (end 142.225 51.625) (width 0.2) (layer "F.Cu") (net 11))
 (segment (start 143.817893 45.475) (end 142.892893 46.4) (width 0.2) (layer "F.Cu") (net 5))
 (segment (start 147.4 46.2) (end 145.925 46.2) (width 0.2) (layer "F.Cu") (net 5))
 (segment (start 142.892893 46.4) (end 142.699973 46.4) (width 0.2) (layer "F.Cu") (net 5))
 (segment (start 145.925 46.2) (end 145.9 46.175) (width 0.2) (layer "F.Cu") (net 5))
 (segment (start 145.9 46.175) (end 145.2 45.475) (width 0.2) (layer "F.Cu") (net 5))
 (segment (start 145.2 45.475) (end 143.817893 45.475) (width 0.2) (layer "F.Cu") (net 5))
 (segment (start 144.3 46.175) (end 143.274999 47.200001) (width 0.2) (layer "F.Cu") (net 8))
 (segment (start 143.274999 47.200001) (end 142.699973 47.200001) (width 0.2) (layer "F.Cu") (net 8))
 (segment (start 147.4 47.8) (end 146.725 47.125) (width 0.2) (layer "F.Cu") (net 8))
 (segment (start 145.25 47.125) (end 144.3 46.175) (width 0.2) (layer "F.Cu") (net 8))
 (segment (start 146.725 47.125) (end 145.25 47.125) (width 0.2) (layer "F.Cu") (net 8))
 (segment (start 152.57 46.5) (end 152.57 44.055) (width 0.2) (layer "F.Cu") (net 7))
 (segment (start 152.65 43.975) (end 152.2875 44.3375) (width 0.2) (layer "F.Cu") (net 7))
 (segment (start 152.57 44.055) (end 152.65 43.975) (width 0.2) (layer "F.Cu") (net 7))
 (segment (start 152.2875 44.3375) (end 150.1 44.3375) (width 0.2) (layer "F.Cu") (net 7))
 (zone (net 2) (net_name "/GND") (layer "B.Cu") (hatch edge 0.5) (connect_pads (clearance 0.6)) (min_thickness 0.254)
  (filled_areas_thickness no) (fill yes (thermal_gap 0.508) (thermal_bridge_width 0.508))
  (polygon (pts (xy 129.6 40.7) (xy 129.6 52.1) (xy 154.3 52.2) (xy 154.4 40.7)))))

